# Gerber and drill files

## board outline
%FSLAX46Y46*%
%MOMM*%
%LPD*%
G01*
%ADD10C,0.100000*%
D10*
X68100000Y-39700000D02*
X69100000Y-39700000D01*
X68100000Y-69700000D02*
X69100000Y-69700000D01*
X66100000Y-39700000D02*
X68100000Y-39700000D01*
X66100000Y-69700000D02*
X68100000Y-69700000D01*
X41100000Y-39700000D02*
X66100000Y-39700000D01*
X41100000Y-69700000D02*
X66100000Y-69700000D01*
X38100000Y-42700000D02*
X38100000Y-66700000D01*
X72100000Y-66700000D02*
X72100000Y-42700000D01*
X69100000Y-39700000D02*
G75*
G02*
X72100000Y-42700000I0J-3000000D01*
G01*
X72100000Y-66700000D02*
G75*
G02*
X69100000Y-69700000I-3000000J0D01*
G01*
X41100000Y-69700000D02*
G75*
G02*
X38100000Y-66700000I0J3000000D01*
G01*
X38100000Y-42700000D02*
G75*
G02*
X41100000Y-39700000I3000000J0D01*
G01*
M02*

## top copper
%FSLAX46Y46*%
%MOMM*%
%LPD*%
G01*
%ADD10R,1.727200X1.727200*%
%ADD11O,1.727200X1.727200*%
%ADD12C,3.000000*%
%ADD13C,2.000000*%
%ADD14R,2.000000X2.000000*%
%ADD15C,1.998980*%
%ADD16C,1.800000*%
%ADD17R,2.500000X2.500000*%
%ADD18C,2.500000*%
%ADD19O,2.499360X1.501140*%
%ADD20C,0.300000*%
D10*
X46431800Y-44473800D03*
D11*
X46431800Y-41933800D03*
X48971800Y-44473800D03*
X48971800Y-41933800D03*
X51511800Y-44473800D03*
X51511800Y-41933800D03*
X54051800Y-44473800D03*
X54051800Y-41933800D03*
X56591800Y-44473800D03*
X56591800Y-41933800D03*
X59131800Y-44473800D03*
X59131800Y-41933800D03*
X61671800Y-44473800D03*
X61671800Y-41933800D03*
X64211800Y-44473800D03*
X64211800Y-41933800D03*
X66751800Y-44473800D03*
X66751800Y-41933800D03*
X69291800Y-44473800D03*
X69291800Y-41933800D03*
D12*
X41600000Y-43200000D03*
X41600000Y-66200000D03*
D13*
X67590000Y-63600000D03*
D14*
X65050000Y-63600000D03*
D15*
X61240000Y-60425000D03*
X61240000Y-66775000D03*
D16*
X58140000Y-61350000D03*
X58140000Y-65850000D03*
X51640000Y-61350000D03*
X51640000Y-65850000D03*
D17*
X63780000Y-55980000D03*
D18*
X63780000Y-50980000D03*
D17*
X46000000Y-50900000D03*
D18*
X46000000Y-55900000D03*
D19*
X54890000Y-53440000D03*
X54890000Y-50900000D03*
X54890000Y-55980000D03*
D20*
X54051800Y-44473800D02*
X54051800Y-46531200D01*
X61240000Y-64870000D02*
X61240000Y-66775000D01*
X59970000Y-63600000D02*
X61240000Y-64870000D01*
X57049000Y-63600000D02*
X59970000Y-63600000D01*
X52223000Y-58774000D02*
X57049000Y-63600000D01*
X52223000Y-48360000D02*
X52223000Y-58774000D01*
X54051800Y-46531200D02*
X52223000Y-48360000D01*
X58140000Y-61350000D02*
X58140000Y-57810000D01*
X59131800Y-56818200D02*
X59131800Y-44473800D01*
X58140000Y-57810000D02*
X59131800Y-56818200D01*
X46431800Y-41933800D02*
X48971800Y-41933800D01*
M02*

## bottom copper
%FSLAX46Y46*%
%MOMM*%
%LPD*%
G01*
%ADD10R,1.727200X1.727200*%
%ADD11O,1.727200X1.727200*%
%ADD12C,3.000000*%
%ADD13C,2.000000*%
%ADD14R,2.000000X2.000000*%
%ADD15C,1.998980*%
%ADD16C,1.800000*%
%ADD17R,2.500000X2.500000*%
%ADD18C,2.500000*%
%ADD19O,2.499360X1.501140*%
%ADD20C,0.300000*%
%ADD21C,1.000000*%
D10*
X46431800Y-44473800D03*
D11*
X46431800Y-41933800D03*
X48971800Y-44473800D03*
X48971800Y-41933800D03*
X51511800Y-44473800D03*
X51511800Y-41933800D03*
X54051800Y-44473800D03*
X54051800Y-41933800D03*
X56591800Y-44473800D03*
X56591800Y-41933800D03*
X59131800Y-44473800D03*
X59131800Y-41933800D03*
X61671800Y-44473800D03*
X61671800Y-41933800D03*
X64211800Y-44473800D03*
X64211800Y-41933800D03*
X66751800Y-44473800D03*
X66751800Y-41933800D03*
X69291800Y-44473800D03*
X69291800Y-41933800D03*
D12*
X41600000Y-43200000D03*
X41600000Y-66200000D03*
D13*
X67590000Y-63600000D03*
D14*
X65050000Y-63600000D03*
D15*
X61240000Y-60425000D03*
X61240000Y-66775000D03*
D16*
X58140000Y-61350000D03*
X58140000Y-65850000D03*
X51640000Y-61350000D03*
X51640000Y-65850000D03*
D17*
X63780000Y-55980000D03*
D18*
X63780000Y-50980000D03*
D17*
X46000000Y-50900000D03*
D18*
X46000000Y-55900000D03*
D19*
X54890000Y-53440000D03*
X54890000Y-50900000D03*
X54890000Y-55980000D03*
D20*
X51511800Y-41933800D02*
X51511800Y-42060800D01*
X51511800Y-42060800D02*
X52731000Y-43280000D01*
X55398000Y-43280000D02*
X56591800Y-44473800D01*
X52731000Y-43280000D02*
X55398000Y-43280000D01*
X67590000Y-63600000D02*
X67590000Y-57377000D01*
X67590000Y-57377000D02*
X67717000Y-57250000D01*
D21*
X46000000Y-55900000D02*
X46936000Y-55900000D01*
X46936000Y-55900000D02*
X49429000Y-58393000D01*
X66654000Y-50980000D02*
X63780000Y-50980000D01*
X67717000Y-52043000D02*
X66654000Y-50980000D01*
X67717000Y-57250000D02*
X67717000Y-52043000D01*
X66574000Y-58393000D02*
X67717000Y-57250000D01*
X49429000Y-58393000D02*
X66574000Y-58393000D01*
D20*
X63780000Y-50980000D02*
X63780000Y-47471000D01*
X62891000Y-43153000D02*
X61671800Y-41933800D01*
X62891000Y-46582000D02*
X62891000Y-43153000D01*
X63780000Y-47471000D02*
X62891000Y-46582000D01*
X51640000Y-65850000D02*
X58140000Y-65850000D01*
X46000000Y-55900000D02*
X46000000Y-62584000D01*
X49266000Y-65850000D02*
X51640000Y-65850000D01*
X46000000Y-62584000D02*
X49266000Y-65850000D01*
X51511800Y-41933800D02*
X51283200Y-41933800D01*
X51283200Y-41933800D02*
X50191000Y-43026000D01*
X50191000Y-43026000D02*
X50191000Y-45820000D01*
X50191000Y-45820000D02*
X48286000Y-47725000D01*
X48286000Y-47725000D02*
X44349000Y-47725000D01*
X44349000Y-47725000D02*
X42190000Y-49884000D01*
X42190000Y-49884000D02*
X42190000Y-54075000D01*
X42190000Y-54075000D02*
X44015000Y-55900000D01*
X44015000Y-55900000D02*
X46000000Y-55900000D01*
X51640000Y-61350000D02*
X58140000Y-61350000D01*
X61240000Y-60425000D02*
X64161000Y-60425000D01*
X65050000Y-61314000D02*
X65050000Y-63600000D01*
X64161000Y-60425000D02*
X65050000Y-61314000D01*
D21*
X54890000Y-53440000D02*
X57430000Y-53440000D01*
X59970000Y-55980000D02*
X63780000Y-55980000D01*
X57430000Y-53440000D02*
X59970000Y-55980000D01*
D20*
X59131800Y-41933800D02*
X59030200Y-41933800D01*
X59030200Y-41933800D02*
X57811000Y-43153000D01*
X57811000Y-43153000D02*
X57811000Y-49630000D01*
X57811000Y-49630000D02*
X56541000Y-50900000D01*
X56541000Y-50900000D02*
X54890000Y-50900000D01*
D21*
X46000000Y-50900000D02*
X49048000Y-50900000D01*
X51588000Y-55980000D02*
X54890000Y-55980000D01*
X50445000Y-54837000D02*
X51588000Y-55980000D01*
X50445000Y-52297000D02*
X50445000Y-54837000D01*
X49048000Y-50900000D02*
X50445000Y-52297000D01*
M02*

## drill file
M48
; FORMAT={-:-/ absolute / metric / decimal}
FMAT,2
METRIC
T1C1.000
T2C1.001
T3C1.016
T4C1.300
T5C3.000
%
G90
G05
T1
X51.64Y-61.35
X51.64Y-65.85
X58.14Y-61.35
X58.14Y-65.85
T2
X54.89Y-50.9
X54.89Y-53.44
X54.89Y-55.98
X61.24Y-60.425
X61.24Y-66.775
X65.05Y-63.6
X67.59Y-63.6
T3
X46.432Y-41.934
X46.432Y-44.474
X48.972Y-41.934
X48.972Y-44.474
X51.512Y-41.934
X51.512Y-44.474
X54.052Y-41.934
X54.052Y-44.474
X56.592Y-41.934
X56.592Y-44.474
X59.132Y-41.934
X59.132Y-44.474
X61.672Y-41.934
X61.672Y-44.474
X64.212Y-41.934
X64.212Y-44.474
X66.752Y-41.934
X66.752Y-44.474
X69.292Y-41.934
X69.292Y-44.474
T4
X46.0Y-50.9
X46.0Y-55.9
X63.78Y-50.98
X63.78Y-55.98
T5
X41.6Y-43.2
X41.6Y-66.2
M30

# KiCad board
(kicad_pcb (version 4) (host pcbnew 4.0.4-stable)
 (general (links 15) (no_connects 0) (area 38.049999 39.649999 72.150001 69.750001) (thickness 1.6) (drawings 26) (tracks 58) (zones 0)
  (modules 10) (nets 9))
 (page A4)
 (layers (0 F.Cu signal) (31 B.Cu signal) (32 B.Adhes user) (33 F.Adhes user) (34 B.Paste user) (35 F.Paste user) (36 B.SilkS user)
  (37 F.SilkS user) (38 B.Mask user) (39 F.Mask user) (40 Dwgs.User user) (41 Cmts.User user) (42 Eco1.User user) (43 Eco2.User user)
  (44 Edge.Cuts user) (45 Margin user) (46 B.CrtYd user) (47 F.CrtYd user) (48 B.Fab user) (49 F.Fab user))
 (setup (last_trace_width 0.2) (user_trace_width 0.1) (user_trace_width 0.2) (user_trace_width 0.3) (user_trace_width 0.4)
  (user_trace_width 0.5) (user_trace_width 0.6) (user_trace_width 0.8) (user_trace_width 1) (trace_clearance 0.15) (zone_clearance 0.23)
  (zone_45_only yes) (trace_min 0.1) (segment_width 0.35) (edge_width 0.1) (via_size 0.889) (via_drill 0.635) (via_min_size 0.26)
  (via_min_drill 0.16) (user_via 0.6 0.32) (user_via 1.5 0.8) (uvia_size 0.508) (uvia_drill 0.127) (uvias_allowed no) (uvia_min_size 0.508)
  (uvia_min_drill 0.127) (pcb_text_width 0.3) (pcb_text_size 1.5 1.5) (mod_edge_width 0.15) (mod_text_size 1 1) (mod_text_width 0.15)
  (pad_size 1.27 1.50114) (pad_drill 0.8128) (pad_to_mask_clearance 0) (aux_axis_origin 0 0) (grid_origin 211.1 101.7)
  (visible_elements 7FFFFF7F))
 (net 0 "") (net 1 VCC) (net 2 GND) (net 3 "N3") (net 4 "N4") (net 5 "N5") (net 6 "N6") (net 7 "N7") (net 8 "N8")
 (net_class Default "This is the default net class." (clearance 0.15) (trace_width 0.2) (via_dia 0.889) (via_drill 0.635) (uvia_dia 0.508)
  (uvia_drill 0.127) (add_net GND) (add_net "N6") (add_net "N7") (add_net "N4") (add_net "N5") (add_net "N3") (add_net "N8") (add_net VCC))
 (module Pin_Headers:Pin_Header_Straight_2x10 (layer F.Cu) (at 46.4318 44.4738 90)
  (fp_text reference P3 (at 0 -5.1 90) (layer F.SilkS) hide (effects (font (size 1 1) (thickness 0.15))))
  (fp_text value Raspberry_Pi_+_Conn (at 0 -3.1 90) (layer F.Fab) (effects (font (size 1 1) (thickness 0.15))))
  (pad 1 thru_hole rect (at 0 0 90) (size 1.7272 1.7272) (drill 1.016) (layers *.Cu *.Mask F.SilkS))
  (pad 2 thru_hole oval (at 2.54 0 90) (size 1.7272 1.7272) (drill 1.016) (layers *.Cu *.Mask F.SilkS) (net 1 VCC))
  (pad 3 thru_hole oval (at 0 2.54 90) (size 1.7272 1.7272) (drill 1.016) (layers *.Cu *.Mask F.SilkS))
  (pad 4 thru_hole oval (at 2.54 2.54 90) (size 1.7272 1.7272) (drill 1.016) (layers *.Cu *.Mask F.SilkS) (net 1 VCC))
  (pad 5 thru_hole oval (at 0 5.08 90) (size 1.7272 1.7272) (drill 1.016) (layers *.Cu *.Mask F.SilkS))
  (pad 6 thru_hole oval (at 2.54 5.08 90) (size 1.7272 1.7272) (drill 1.016) (layers *.Cu *.Mask F.SilkS) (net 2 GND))
  (pad 7 thru_hole oval (at 0 7.62 90) (size 1.7272 1.7272) (drill 1.016) (layers *.Cu *.Mask F.SilkS) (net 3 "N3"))
  (pad 8 thru_hole oval (at 2.54 7.62 90) (size 1.7272 1.7272) (drill 1.016) (layers *.Cu *.Mask F.SilkS))
  (pad 9 thru_hole oval (at 0 10.16 90) (size 1.7272 1.7272) (drill 1.016) (layers *.Cu *.Mask F.SilkS) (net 2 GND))
  (pad 10 thru_hole oval (at 2.54 10.16 90) (size 1.7272 1.7272) (drill 1.016) (layers *.Cu *.Mask F.SilkS))
  (pad 11 thru_hole oval (at 0 12.7 90) (size 1.7272 1.7272) (drill 1.016) (layers *.Cu *.Mask F.SilkS) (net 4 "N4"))
  (pad 12 thru_hole oval (at 2.54 12.7 90) (size 1.7272 1.7272) (drill 1.016) (layers *.Cu *.Mask F.SilkS) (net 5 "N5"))
  (pad 13 thru_hole oval (at 0 15.24 90) (size 1.7272 1.7272) (drill 1.016) (layers *.Cu *.Mask F.SilkS))
  (pad 14 thru_hole oval (at 2.54 15.24 90) (size 1.7272 1.7272) (drill 1.016) (layers *.Cu *.Mask F.SilkS) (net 2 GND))
  (pad 15 thru_hole oval (at 0 17.78 90) (size 1.7272 1.7272) (drill 1.016) (layers *.Cu *.Mask F.SilkS))
  (pad 16 thru_hole oval (at 2.54 17.78 90) (size 1.7272 1.7272) (drill 1.016) (layers *.Cu *.Mask F.SilkS))
  (pad 17 thru_hole oval (at 0 20.32 90) (size 1.7272 1.7272) (drill 1.016) (layers *.Cu *.Mask F.SilkS))
  (pad 18 thru_hole oval (at 2.54 20.32 90) (size 1.7272 1.7272) (drill 1.016) (layers *.Cu *.Mask F.SilkS))
  (pad 19 thru_hole oval (at 0 22.86 90) (size 1.7272 1.7272) (drill 1.016) (layers *.Cu *.Mask F.SilkS))
  (pad 20 thru_hole oval (at 2.54 22.86 90) (size 1.7272 1.7272) (drill 1.016) (layers *.Cu *.Mask F.SilkS)))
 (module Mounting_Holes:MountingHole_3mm (layer F.Cu) (at 41.6 43.2)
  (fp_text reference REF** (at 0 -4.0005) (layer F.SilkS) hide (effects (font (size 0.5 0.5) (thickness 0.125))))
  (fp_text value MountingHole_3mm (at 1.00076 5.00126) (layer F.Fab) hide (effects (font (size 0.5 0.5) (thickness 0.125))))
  (pad 1 thru_hole circle (at 0 0) (size 3 3) (drill 3) (layers)))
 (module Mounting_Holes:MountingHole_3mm (layer F.Cu) (at 41.6 66.2)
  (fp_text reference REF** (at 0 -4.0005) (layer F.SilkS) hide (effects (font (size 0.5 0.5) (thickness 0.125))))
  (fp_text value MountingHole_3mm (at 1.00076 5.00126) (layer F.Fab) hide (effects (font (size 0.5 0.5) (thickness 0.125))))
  (pad 1 thru_hole circle (at 0 0) (size 3 3) (drill 3) (layers)))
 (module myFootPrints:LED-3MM (layer F.Cu) (at 67.59 63.6 180)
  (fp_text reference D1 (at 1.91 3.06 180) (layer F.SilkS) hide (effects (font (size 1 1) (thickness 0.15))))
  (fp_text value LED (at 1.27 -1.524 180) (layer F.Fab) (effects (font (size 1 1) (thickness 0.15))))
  (pad 1 thru_hole circle (at 0 0 270) (size 2 2) (drill 1.00076) (layers *.Cu B.Mask) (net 2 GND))
  (pad 2 thru_hole rect (at 2.54 0 180) (size 2 2) (drill 1.00076) (layers *.Cu B.Mask) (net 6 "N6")))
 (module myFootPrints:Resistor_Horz (layer F.Cu) (at 61.24 63.6 270)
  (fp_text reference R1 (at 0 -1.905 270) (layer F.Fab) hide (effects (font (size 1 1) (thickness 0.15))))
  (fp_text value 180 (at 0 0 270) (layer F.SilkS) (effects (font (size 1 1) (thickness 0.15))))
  (pad 1 thru_hole circle (at -3.175 0 270) (size 1.99898 1.99898) (drill 1.00076) (layers *.Cu *.SilkS *.Mask) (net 6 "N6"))
  (pad 2 thru_hole circle (at 3.175 0 270) (size 1.99898 1.99898) (drill 1.00076) (layers *.Cu *.SilkS *.Mask) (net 3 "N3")))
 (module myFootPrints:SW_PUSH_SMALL (layer F.Cu) (at 54.89 63.6)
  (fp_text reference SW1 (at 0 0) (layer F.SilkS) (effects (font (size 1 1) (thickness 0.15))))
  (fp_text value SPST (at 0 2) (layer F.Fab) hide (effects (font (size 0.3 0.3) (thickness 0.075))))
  (pad 1 thru_hole circle (at 3.25 -2.25) (size 1.8 1.8) (drill 1) (layers *.Cu B.Mask) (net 4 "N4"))
  (pad 2 thru_hole circle (at 3.25 2.25) (size 1.8 1.8) (drill 1) (layers *.Cu B.Mask) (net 2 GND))
  (pad 1 thru_hole circle (at -3.25 -2.25) (size 1.8 1.8) (drill 1) (layers *.Cu B.Mask) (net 4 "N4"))
  (pad 2 thru_hole circle (at -3.25 2.25) (size 1.8 1.8) (drill 1) (layers *.Cu B.Mask) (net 2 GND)))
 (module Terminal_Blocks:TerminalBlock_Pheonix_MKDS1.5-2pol (layer F.Cu) (at 63.78 55.98 90)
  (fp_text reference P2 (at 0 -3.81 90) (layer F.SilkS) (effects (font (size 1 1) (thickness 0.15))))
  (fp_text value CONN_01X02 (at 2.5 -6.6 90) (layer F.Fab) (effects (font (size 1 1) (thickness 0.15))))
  (pad 1 thru_hole rect (at 0 0 90) (size 2.5 2.5) (drill 1.3) (layers *.Cu *.Mask F.SilkS) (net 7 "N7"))
  (pad 2 thru_hole circle (at 5 0 90) (size 2.5 2.5) (drill 1.3) (layers *.Cu *.Mask F.SilkS) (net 2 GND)))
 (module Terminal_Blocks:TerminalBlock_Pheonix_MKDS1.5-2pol (layer F.Cu) (at 46 50.9 270)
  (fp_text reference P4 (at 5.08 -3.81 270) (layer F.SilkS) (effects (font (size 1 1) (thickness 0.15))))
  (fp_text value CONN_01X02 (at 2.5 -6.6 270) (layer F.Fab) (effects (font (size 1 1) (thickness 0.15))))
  (pad 1 thru_hole rect (at 0 0 270) (size 2.5 2.5) (drill 1.3) (layers *.Cu *.Mask F.SilkS) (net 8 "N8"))
  (pad 2 thru_hole circle (at 5 0 270) (size 2.5 2.5) (drill 1.3) (layers *.Cu *.Mask F.SilkS) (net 2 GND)))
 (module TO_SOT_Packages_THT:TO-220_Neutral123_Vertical (layer F.Cu) (at 54.89 53.44 270)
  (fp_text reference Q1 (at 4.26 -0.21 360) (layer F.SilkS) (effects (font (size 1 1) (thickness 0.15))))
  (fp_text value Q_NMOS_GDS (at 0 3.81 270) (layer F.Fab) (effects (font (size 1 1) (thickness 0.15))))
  (pad 2 thru_hole oval (at 0 0) (size 2.49936 1.50114) (drill 1.00076) (layers *.Cu *.Mask F.SilkS) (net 7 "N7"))
  (pad 1 thru_hole oval (at -2.54 0) (size 2.49936 1.50114) (drill 1.00076) (layers *.Cu *.Mask F.SilkS) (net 5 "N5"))
  (pad 3 thru_hole oval (at 2.54 0) (size 2.49936 1.50114) (drill 1.00076) (layers *.Cu *.Mask F.SilkS) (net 8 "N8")))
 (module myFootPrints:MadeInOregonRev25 (layer F.Cu) (at 46.508 62.584)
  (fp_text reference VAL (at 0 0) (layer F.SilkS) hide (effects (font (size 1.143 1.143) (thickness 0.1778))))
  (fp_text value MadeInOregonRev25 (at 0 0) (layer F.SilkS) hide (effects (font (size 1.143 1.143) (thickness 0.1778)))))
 (gr_line (start 68.1 39.7) (end 69.1 39.7) (angle 90) (layer Edge.Cuts) (width 0.1))
 (gr_line (start 68.1 69.7) (end 69.1 69.7) (angle 90) (layer Edge.Cuts) (width 0.1))
 (gr_line (start 66.1 39.7) (end 68.1 39.7) (angle 90) (layer Edge.Cuts) (width 0.1))
 (gr_line (start 66.1 69.7) (end 68.1 69.7) (angle 90) (layer Edge.Cuts) (width 0.1))
 (gr_line (start 41.1 39.7) (end 66.1 39.7) (angle 90) (layer Edge.Cuts) (width 0.1))
 (gr_line (start 41.1 69.7) (end 66.1 69.7) (angle 90) (layer Edge.Cuts) (width 0.1))
 (gr_line (start 38.1 42.7) (end 38.1 66.7) (angle 90) (layer Edge.Cuts) (width 0.1))
 (gr_line (start 72.1 66.7) (end 72.1 42.7) (angle 90) (layer Edge.Cuts) (width 0.1))
 (gr_arc (start 69.1 42.7) (end 69.1 39.7) (angle 90) (layer Edge.Cuts) (width 0.1))
 (gr_arc (start 69.1 66.7) (end 72.1 66.7) (angle 90) (layer Edge.Cuts) (width 0.1))
 (gr_arc (start 41.1 66.7) (end 41.1 69.7) (angle 90) (layer Edge.Cuts) (width 0.1))
 (gr_arc (start 41.1 42.7) (end 38.1 42.7) (angle 90) (layer Edge.Cuts) (width 0.1))
 (segment (start 51.5118 41.9338) (end 51.5118 42.0608) (width 0.3) (layer B.Cu) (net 2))
 (segment (start 51.5118 42.0608) (end 52.731 43.28) (width 0.3) (layer B.Cu) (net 2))
 (segment (start 55.398 43.28) (end 56.5918 44.4738) (width 0.3) (layer B.Cu) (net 2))
 (segment (start 52.731 43.28) (end 55.398 43.28) (width 0.3) (layer B.Cu) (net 2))
 (segment (start 67.59 63.6) (end 67.59 57.377) (width 0.3) (layer B.Cu) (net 2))
 (segment (start 67.59 57.377) (end 67.717 57.25) (width 0.3) (layer B.Cu) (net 2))
 (segment (start 46 55.9) (end 46.936 55.9) (width 1) (layer B.Cu) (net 2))
 (segment (start 46.936 55.9) (end 49.429 58.393) (width 1) (layer B.Cu) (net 2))
 (segment (start 66.654 50.98) (end 63.78 50.98) (width 1) (layer B.Cu) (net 2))
 (segment (start 67.717 52.043) (end 66.654 50.98) (width 1) (layer B.Cu) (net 2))
 (segment (start 67.717 57.25) (end 67.717 52.043) (width 1) (layer B.Cu) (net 2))
 (segment (start 66.574 58.393) (end 67.717 57.25) (width 1) (layer B.Cu) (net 2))
 (segment (start 49.429 58.393) (end 66.574 58.393) (width 1) (layer B.Cu) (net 2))
 (segment (start 63.78 50.98) (end 63.78 47.471) (width 0.3) (layer B.Cu) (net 2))
 (segment (start 62.891 43.153) (end 61.6718 41.9338) (width 0.3) (layer B.Cu) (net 2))
 (segment (start 62.891 46.582) (end 62.891 43.153) (width 0.3) (layer B.Cu) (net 2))
 (segment (start 63.78 47.471) (end 62.891 46.582) (width 0.3) (layer B.Cu) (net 2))
 (segment (start 51.64 65.85) (end 58.14 65.85) (width 0.3) (layer B.Cu) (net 2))
 (segment (start 46 55.9) (end 46 62.584) (width 0.3) (layer B.Cu) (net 2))
 (segment (start 49.266 65.85) (end 51.64 65.85) (width 0.3) (layer B.Cu) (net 2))
 (segment (start 46 62.584) (end 49.266 65.85) (width 0.3) (layer B.Cu) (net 2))
 (segment (start 51.5118 41.9338) (end 51.2832 41.9338) (width 0.3) (layer B.Cu) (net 2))
 (segment (start 51.2832 41.9338) (end 50.191 43.026) (width 0.3) (layer B.Cu) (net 2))
 (segment (start 50.191 43.026) (end 50.191 45.82) (width 0.3) (layer B.Cu) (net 2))
 (segment (start 50.191 45.82) (end 48.286 47.725) (width 0.3) (layer B.Cu) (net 2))
 (segment (start 48.286 47.725) (end 44.349 47.725) (width 0.3) (layer B.Cu) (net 2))
 (segment (start 44.349 47.725) (end 42.19 49.884) (width 0.3) (layer B.Cu) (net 2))
 (segment (start 42.19 49.884) (end 42.19 54.075) (width 0.3) (layer B.Cu) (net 2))
 (segment (start 42.19 54.075) (end 44.015 55.9) (width 0.3) (layer B.Cu) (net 2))
 (segment (start 44.015 55.9) (end 46 55.9) (width 0.3) (layer B.Cu) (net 2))
 (segment (start 54.0518 44.4738) (end 54.0518 46.5312) (width 0.3) (layer F.Cu) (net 3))
 (segment (start 61.24 64.87) (end 61.24 66.775) (width 0.3) (layer F.Cu) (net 3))
 (segment (start 59.97 63.6) (end 61.24 64.87) (width 0.3) (layer F.Cu) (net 3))
 (segment (start 57.049 63.6) (end 59.97 63.6) (width 0.3) (layer F.Cu) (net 3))
 (segment (start 52.223 58.774) (end 57.049 63.6) (width 0.3) (layer F.Cu) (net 3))
 (segment (start 52.223 48.36) (end 52.223 58.774) (width 0.3) (layer F.Cu) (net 3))
 (segment (start 54.0518 46.5312) (end 52.223 48.36) (width 0.3) (layer F.Cu) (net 3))
 (segment (start 58.14 61.35) (end 58.14 57.81) (width 0.3) (layer F.Cu) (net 4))
 (segment (start 59.1318 56.8182) (end 59.1318 44.4738) (width 0.3) (layer F.Cu) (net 4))
 (segment (start 58.14 57.81) (end 59.1318 56.8182) (width 0.3) (layer F.Cu) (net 4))
 (segment (start 51.64 61.35) (end 58.14 61.35) (width 0.3) (layer B.Cu) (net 4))
 (segment (start 46.4318 41.9338) (end 48.9718 41.9338) (width 0.3) (layer F.Cu) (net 1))
 (segment (start 61.24 60.425) (end 64.161 60.425) (width 0.3) (layer B.Cu) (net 6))
 (segment (start 65.05 61.314) (end 65.05 63.6) (width 0.3) (layer B.Cu) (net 6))
 (segment (start 64.161 60.425) (end 65.05 61.314) (width 0.3) (layer B.Cu) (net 6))
 (segment (start 54.89 53.44) (end 57.43 53.44) (width 1) (layer B.Cu) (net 7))
 (segment (start 59.97 55.98) (end 63.78 55.98) (width 1) (layer B.Cu) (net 7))
 (segment (start 57.43 53.44) (end 59.97 55.98) (width 1) (layer B.Cu) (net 7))
 (segment (start 59.1318 41.9338) (end 59.0302 41.9338) (width 0.3) (layer B.Cu) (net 5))
 (segment (start 59.0302 41.9338) (end 57.811 43.153) (width 0.3) (layer B.Cu) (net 5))
 (segment (start 57.811 43.153) (end 57.811 49.63) (width 0.3) (layer B.Cu) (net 5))
 (segment (start 57.811 49.63) (end 56.541 50.9) (width 0.3) (layer B.Cu) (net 5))
 (segment (start 56.541 50.9) (end 54.89 50.9) (width 0.3) (layer B.Cu) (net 5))
 (segment (start 46 50.9) (end 49.048 50.9) (width 1) (layer B.Cu) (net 8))
 (segment (start 51.588 55.98) (end 54.89 55.98) (width 1) (layer B.Cu) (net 8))
 (segment (start 50.445 54.837) (end 51.588 55.98) (width 1) (layer B.Cu) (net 8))
 (segment (start 50.445 52.297) (end 50.445 54.837) (width 1) (layer B.Cu) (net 8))
 (segment (start 49.048 50.9) (end 50.445 52.297) (width 1) (layer B.Cu) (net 8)))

